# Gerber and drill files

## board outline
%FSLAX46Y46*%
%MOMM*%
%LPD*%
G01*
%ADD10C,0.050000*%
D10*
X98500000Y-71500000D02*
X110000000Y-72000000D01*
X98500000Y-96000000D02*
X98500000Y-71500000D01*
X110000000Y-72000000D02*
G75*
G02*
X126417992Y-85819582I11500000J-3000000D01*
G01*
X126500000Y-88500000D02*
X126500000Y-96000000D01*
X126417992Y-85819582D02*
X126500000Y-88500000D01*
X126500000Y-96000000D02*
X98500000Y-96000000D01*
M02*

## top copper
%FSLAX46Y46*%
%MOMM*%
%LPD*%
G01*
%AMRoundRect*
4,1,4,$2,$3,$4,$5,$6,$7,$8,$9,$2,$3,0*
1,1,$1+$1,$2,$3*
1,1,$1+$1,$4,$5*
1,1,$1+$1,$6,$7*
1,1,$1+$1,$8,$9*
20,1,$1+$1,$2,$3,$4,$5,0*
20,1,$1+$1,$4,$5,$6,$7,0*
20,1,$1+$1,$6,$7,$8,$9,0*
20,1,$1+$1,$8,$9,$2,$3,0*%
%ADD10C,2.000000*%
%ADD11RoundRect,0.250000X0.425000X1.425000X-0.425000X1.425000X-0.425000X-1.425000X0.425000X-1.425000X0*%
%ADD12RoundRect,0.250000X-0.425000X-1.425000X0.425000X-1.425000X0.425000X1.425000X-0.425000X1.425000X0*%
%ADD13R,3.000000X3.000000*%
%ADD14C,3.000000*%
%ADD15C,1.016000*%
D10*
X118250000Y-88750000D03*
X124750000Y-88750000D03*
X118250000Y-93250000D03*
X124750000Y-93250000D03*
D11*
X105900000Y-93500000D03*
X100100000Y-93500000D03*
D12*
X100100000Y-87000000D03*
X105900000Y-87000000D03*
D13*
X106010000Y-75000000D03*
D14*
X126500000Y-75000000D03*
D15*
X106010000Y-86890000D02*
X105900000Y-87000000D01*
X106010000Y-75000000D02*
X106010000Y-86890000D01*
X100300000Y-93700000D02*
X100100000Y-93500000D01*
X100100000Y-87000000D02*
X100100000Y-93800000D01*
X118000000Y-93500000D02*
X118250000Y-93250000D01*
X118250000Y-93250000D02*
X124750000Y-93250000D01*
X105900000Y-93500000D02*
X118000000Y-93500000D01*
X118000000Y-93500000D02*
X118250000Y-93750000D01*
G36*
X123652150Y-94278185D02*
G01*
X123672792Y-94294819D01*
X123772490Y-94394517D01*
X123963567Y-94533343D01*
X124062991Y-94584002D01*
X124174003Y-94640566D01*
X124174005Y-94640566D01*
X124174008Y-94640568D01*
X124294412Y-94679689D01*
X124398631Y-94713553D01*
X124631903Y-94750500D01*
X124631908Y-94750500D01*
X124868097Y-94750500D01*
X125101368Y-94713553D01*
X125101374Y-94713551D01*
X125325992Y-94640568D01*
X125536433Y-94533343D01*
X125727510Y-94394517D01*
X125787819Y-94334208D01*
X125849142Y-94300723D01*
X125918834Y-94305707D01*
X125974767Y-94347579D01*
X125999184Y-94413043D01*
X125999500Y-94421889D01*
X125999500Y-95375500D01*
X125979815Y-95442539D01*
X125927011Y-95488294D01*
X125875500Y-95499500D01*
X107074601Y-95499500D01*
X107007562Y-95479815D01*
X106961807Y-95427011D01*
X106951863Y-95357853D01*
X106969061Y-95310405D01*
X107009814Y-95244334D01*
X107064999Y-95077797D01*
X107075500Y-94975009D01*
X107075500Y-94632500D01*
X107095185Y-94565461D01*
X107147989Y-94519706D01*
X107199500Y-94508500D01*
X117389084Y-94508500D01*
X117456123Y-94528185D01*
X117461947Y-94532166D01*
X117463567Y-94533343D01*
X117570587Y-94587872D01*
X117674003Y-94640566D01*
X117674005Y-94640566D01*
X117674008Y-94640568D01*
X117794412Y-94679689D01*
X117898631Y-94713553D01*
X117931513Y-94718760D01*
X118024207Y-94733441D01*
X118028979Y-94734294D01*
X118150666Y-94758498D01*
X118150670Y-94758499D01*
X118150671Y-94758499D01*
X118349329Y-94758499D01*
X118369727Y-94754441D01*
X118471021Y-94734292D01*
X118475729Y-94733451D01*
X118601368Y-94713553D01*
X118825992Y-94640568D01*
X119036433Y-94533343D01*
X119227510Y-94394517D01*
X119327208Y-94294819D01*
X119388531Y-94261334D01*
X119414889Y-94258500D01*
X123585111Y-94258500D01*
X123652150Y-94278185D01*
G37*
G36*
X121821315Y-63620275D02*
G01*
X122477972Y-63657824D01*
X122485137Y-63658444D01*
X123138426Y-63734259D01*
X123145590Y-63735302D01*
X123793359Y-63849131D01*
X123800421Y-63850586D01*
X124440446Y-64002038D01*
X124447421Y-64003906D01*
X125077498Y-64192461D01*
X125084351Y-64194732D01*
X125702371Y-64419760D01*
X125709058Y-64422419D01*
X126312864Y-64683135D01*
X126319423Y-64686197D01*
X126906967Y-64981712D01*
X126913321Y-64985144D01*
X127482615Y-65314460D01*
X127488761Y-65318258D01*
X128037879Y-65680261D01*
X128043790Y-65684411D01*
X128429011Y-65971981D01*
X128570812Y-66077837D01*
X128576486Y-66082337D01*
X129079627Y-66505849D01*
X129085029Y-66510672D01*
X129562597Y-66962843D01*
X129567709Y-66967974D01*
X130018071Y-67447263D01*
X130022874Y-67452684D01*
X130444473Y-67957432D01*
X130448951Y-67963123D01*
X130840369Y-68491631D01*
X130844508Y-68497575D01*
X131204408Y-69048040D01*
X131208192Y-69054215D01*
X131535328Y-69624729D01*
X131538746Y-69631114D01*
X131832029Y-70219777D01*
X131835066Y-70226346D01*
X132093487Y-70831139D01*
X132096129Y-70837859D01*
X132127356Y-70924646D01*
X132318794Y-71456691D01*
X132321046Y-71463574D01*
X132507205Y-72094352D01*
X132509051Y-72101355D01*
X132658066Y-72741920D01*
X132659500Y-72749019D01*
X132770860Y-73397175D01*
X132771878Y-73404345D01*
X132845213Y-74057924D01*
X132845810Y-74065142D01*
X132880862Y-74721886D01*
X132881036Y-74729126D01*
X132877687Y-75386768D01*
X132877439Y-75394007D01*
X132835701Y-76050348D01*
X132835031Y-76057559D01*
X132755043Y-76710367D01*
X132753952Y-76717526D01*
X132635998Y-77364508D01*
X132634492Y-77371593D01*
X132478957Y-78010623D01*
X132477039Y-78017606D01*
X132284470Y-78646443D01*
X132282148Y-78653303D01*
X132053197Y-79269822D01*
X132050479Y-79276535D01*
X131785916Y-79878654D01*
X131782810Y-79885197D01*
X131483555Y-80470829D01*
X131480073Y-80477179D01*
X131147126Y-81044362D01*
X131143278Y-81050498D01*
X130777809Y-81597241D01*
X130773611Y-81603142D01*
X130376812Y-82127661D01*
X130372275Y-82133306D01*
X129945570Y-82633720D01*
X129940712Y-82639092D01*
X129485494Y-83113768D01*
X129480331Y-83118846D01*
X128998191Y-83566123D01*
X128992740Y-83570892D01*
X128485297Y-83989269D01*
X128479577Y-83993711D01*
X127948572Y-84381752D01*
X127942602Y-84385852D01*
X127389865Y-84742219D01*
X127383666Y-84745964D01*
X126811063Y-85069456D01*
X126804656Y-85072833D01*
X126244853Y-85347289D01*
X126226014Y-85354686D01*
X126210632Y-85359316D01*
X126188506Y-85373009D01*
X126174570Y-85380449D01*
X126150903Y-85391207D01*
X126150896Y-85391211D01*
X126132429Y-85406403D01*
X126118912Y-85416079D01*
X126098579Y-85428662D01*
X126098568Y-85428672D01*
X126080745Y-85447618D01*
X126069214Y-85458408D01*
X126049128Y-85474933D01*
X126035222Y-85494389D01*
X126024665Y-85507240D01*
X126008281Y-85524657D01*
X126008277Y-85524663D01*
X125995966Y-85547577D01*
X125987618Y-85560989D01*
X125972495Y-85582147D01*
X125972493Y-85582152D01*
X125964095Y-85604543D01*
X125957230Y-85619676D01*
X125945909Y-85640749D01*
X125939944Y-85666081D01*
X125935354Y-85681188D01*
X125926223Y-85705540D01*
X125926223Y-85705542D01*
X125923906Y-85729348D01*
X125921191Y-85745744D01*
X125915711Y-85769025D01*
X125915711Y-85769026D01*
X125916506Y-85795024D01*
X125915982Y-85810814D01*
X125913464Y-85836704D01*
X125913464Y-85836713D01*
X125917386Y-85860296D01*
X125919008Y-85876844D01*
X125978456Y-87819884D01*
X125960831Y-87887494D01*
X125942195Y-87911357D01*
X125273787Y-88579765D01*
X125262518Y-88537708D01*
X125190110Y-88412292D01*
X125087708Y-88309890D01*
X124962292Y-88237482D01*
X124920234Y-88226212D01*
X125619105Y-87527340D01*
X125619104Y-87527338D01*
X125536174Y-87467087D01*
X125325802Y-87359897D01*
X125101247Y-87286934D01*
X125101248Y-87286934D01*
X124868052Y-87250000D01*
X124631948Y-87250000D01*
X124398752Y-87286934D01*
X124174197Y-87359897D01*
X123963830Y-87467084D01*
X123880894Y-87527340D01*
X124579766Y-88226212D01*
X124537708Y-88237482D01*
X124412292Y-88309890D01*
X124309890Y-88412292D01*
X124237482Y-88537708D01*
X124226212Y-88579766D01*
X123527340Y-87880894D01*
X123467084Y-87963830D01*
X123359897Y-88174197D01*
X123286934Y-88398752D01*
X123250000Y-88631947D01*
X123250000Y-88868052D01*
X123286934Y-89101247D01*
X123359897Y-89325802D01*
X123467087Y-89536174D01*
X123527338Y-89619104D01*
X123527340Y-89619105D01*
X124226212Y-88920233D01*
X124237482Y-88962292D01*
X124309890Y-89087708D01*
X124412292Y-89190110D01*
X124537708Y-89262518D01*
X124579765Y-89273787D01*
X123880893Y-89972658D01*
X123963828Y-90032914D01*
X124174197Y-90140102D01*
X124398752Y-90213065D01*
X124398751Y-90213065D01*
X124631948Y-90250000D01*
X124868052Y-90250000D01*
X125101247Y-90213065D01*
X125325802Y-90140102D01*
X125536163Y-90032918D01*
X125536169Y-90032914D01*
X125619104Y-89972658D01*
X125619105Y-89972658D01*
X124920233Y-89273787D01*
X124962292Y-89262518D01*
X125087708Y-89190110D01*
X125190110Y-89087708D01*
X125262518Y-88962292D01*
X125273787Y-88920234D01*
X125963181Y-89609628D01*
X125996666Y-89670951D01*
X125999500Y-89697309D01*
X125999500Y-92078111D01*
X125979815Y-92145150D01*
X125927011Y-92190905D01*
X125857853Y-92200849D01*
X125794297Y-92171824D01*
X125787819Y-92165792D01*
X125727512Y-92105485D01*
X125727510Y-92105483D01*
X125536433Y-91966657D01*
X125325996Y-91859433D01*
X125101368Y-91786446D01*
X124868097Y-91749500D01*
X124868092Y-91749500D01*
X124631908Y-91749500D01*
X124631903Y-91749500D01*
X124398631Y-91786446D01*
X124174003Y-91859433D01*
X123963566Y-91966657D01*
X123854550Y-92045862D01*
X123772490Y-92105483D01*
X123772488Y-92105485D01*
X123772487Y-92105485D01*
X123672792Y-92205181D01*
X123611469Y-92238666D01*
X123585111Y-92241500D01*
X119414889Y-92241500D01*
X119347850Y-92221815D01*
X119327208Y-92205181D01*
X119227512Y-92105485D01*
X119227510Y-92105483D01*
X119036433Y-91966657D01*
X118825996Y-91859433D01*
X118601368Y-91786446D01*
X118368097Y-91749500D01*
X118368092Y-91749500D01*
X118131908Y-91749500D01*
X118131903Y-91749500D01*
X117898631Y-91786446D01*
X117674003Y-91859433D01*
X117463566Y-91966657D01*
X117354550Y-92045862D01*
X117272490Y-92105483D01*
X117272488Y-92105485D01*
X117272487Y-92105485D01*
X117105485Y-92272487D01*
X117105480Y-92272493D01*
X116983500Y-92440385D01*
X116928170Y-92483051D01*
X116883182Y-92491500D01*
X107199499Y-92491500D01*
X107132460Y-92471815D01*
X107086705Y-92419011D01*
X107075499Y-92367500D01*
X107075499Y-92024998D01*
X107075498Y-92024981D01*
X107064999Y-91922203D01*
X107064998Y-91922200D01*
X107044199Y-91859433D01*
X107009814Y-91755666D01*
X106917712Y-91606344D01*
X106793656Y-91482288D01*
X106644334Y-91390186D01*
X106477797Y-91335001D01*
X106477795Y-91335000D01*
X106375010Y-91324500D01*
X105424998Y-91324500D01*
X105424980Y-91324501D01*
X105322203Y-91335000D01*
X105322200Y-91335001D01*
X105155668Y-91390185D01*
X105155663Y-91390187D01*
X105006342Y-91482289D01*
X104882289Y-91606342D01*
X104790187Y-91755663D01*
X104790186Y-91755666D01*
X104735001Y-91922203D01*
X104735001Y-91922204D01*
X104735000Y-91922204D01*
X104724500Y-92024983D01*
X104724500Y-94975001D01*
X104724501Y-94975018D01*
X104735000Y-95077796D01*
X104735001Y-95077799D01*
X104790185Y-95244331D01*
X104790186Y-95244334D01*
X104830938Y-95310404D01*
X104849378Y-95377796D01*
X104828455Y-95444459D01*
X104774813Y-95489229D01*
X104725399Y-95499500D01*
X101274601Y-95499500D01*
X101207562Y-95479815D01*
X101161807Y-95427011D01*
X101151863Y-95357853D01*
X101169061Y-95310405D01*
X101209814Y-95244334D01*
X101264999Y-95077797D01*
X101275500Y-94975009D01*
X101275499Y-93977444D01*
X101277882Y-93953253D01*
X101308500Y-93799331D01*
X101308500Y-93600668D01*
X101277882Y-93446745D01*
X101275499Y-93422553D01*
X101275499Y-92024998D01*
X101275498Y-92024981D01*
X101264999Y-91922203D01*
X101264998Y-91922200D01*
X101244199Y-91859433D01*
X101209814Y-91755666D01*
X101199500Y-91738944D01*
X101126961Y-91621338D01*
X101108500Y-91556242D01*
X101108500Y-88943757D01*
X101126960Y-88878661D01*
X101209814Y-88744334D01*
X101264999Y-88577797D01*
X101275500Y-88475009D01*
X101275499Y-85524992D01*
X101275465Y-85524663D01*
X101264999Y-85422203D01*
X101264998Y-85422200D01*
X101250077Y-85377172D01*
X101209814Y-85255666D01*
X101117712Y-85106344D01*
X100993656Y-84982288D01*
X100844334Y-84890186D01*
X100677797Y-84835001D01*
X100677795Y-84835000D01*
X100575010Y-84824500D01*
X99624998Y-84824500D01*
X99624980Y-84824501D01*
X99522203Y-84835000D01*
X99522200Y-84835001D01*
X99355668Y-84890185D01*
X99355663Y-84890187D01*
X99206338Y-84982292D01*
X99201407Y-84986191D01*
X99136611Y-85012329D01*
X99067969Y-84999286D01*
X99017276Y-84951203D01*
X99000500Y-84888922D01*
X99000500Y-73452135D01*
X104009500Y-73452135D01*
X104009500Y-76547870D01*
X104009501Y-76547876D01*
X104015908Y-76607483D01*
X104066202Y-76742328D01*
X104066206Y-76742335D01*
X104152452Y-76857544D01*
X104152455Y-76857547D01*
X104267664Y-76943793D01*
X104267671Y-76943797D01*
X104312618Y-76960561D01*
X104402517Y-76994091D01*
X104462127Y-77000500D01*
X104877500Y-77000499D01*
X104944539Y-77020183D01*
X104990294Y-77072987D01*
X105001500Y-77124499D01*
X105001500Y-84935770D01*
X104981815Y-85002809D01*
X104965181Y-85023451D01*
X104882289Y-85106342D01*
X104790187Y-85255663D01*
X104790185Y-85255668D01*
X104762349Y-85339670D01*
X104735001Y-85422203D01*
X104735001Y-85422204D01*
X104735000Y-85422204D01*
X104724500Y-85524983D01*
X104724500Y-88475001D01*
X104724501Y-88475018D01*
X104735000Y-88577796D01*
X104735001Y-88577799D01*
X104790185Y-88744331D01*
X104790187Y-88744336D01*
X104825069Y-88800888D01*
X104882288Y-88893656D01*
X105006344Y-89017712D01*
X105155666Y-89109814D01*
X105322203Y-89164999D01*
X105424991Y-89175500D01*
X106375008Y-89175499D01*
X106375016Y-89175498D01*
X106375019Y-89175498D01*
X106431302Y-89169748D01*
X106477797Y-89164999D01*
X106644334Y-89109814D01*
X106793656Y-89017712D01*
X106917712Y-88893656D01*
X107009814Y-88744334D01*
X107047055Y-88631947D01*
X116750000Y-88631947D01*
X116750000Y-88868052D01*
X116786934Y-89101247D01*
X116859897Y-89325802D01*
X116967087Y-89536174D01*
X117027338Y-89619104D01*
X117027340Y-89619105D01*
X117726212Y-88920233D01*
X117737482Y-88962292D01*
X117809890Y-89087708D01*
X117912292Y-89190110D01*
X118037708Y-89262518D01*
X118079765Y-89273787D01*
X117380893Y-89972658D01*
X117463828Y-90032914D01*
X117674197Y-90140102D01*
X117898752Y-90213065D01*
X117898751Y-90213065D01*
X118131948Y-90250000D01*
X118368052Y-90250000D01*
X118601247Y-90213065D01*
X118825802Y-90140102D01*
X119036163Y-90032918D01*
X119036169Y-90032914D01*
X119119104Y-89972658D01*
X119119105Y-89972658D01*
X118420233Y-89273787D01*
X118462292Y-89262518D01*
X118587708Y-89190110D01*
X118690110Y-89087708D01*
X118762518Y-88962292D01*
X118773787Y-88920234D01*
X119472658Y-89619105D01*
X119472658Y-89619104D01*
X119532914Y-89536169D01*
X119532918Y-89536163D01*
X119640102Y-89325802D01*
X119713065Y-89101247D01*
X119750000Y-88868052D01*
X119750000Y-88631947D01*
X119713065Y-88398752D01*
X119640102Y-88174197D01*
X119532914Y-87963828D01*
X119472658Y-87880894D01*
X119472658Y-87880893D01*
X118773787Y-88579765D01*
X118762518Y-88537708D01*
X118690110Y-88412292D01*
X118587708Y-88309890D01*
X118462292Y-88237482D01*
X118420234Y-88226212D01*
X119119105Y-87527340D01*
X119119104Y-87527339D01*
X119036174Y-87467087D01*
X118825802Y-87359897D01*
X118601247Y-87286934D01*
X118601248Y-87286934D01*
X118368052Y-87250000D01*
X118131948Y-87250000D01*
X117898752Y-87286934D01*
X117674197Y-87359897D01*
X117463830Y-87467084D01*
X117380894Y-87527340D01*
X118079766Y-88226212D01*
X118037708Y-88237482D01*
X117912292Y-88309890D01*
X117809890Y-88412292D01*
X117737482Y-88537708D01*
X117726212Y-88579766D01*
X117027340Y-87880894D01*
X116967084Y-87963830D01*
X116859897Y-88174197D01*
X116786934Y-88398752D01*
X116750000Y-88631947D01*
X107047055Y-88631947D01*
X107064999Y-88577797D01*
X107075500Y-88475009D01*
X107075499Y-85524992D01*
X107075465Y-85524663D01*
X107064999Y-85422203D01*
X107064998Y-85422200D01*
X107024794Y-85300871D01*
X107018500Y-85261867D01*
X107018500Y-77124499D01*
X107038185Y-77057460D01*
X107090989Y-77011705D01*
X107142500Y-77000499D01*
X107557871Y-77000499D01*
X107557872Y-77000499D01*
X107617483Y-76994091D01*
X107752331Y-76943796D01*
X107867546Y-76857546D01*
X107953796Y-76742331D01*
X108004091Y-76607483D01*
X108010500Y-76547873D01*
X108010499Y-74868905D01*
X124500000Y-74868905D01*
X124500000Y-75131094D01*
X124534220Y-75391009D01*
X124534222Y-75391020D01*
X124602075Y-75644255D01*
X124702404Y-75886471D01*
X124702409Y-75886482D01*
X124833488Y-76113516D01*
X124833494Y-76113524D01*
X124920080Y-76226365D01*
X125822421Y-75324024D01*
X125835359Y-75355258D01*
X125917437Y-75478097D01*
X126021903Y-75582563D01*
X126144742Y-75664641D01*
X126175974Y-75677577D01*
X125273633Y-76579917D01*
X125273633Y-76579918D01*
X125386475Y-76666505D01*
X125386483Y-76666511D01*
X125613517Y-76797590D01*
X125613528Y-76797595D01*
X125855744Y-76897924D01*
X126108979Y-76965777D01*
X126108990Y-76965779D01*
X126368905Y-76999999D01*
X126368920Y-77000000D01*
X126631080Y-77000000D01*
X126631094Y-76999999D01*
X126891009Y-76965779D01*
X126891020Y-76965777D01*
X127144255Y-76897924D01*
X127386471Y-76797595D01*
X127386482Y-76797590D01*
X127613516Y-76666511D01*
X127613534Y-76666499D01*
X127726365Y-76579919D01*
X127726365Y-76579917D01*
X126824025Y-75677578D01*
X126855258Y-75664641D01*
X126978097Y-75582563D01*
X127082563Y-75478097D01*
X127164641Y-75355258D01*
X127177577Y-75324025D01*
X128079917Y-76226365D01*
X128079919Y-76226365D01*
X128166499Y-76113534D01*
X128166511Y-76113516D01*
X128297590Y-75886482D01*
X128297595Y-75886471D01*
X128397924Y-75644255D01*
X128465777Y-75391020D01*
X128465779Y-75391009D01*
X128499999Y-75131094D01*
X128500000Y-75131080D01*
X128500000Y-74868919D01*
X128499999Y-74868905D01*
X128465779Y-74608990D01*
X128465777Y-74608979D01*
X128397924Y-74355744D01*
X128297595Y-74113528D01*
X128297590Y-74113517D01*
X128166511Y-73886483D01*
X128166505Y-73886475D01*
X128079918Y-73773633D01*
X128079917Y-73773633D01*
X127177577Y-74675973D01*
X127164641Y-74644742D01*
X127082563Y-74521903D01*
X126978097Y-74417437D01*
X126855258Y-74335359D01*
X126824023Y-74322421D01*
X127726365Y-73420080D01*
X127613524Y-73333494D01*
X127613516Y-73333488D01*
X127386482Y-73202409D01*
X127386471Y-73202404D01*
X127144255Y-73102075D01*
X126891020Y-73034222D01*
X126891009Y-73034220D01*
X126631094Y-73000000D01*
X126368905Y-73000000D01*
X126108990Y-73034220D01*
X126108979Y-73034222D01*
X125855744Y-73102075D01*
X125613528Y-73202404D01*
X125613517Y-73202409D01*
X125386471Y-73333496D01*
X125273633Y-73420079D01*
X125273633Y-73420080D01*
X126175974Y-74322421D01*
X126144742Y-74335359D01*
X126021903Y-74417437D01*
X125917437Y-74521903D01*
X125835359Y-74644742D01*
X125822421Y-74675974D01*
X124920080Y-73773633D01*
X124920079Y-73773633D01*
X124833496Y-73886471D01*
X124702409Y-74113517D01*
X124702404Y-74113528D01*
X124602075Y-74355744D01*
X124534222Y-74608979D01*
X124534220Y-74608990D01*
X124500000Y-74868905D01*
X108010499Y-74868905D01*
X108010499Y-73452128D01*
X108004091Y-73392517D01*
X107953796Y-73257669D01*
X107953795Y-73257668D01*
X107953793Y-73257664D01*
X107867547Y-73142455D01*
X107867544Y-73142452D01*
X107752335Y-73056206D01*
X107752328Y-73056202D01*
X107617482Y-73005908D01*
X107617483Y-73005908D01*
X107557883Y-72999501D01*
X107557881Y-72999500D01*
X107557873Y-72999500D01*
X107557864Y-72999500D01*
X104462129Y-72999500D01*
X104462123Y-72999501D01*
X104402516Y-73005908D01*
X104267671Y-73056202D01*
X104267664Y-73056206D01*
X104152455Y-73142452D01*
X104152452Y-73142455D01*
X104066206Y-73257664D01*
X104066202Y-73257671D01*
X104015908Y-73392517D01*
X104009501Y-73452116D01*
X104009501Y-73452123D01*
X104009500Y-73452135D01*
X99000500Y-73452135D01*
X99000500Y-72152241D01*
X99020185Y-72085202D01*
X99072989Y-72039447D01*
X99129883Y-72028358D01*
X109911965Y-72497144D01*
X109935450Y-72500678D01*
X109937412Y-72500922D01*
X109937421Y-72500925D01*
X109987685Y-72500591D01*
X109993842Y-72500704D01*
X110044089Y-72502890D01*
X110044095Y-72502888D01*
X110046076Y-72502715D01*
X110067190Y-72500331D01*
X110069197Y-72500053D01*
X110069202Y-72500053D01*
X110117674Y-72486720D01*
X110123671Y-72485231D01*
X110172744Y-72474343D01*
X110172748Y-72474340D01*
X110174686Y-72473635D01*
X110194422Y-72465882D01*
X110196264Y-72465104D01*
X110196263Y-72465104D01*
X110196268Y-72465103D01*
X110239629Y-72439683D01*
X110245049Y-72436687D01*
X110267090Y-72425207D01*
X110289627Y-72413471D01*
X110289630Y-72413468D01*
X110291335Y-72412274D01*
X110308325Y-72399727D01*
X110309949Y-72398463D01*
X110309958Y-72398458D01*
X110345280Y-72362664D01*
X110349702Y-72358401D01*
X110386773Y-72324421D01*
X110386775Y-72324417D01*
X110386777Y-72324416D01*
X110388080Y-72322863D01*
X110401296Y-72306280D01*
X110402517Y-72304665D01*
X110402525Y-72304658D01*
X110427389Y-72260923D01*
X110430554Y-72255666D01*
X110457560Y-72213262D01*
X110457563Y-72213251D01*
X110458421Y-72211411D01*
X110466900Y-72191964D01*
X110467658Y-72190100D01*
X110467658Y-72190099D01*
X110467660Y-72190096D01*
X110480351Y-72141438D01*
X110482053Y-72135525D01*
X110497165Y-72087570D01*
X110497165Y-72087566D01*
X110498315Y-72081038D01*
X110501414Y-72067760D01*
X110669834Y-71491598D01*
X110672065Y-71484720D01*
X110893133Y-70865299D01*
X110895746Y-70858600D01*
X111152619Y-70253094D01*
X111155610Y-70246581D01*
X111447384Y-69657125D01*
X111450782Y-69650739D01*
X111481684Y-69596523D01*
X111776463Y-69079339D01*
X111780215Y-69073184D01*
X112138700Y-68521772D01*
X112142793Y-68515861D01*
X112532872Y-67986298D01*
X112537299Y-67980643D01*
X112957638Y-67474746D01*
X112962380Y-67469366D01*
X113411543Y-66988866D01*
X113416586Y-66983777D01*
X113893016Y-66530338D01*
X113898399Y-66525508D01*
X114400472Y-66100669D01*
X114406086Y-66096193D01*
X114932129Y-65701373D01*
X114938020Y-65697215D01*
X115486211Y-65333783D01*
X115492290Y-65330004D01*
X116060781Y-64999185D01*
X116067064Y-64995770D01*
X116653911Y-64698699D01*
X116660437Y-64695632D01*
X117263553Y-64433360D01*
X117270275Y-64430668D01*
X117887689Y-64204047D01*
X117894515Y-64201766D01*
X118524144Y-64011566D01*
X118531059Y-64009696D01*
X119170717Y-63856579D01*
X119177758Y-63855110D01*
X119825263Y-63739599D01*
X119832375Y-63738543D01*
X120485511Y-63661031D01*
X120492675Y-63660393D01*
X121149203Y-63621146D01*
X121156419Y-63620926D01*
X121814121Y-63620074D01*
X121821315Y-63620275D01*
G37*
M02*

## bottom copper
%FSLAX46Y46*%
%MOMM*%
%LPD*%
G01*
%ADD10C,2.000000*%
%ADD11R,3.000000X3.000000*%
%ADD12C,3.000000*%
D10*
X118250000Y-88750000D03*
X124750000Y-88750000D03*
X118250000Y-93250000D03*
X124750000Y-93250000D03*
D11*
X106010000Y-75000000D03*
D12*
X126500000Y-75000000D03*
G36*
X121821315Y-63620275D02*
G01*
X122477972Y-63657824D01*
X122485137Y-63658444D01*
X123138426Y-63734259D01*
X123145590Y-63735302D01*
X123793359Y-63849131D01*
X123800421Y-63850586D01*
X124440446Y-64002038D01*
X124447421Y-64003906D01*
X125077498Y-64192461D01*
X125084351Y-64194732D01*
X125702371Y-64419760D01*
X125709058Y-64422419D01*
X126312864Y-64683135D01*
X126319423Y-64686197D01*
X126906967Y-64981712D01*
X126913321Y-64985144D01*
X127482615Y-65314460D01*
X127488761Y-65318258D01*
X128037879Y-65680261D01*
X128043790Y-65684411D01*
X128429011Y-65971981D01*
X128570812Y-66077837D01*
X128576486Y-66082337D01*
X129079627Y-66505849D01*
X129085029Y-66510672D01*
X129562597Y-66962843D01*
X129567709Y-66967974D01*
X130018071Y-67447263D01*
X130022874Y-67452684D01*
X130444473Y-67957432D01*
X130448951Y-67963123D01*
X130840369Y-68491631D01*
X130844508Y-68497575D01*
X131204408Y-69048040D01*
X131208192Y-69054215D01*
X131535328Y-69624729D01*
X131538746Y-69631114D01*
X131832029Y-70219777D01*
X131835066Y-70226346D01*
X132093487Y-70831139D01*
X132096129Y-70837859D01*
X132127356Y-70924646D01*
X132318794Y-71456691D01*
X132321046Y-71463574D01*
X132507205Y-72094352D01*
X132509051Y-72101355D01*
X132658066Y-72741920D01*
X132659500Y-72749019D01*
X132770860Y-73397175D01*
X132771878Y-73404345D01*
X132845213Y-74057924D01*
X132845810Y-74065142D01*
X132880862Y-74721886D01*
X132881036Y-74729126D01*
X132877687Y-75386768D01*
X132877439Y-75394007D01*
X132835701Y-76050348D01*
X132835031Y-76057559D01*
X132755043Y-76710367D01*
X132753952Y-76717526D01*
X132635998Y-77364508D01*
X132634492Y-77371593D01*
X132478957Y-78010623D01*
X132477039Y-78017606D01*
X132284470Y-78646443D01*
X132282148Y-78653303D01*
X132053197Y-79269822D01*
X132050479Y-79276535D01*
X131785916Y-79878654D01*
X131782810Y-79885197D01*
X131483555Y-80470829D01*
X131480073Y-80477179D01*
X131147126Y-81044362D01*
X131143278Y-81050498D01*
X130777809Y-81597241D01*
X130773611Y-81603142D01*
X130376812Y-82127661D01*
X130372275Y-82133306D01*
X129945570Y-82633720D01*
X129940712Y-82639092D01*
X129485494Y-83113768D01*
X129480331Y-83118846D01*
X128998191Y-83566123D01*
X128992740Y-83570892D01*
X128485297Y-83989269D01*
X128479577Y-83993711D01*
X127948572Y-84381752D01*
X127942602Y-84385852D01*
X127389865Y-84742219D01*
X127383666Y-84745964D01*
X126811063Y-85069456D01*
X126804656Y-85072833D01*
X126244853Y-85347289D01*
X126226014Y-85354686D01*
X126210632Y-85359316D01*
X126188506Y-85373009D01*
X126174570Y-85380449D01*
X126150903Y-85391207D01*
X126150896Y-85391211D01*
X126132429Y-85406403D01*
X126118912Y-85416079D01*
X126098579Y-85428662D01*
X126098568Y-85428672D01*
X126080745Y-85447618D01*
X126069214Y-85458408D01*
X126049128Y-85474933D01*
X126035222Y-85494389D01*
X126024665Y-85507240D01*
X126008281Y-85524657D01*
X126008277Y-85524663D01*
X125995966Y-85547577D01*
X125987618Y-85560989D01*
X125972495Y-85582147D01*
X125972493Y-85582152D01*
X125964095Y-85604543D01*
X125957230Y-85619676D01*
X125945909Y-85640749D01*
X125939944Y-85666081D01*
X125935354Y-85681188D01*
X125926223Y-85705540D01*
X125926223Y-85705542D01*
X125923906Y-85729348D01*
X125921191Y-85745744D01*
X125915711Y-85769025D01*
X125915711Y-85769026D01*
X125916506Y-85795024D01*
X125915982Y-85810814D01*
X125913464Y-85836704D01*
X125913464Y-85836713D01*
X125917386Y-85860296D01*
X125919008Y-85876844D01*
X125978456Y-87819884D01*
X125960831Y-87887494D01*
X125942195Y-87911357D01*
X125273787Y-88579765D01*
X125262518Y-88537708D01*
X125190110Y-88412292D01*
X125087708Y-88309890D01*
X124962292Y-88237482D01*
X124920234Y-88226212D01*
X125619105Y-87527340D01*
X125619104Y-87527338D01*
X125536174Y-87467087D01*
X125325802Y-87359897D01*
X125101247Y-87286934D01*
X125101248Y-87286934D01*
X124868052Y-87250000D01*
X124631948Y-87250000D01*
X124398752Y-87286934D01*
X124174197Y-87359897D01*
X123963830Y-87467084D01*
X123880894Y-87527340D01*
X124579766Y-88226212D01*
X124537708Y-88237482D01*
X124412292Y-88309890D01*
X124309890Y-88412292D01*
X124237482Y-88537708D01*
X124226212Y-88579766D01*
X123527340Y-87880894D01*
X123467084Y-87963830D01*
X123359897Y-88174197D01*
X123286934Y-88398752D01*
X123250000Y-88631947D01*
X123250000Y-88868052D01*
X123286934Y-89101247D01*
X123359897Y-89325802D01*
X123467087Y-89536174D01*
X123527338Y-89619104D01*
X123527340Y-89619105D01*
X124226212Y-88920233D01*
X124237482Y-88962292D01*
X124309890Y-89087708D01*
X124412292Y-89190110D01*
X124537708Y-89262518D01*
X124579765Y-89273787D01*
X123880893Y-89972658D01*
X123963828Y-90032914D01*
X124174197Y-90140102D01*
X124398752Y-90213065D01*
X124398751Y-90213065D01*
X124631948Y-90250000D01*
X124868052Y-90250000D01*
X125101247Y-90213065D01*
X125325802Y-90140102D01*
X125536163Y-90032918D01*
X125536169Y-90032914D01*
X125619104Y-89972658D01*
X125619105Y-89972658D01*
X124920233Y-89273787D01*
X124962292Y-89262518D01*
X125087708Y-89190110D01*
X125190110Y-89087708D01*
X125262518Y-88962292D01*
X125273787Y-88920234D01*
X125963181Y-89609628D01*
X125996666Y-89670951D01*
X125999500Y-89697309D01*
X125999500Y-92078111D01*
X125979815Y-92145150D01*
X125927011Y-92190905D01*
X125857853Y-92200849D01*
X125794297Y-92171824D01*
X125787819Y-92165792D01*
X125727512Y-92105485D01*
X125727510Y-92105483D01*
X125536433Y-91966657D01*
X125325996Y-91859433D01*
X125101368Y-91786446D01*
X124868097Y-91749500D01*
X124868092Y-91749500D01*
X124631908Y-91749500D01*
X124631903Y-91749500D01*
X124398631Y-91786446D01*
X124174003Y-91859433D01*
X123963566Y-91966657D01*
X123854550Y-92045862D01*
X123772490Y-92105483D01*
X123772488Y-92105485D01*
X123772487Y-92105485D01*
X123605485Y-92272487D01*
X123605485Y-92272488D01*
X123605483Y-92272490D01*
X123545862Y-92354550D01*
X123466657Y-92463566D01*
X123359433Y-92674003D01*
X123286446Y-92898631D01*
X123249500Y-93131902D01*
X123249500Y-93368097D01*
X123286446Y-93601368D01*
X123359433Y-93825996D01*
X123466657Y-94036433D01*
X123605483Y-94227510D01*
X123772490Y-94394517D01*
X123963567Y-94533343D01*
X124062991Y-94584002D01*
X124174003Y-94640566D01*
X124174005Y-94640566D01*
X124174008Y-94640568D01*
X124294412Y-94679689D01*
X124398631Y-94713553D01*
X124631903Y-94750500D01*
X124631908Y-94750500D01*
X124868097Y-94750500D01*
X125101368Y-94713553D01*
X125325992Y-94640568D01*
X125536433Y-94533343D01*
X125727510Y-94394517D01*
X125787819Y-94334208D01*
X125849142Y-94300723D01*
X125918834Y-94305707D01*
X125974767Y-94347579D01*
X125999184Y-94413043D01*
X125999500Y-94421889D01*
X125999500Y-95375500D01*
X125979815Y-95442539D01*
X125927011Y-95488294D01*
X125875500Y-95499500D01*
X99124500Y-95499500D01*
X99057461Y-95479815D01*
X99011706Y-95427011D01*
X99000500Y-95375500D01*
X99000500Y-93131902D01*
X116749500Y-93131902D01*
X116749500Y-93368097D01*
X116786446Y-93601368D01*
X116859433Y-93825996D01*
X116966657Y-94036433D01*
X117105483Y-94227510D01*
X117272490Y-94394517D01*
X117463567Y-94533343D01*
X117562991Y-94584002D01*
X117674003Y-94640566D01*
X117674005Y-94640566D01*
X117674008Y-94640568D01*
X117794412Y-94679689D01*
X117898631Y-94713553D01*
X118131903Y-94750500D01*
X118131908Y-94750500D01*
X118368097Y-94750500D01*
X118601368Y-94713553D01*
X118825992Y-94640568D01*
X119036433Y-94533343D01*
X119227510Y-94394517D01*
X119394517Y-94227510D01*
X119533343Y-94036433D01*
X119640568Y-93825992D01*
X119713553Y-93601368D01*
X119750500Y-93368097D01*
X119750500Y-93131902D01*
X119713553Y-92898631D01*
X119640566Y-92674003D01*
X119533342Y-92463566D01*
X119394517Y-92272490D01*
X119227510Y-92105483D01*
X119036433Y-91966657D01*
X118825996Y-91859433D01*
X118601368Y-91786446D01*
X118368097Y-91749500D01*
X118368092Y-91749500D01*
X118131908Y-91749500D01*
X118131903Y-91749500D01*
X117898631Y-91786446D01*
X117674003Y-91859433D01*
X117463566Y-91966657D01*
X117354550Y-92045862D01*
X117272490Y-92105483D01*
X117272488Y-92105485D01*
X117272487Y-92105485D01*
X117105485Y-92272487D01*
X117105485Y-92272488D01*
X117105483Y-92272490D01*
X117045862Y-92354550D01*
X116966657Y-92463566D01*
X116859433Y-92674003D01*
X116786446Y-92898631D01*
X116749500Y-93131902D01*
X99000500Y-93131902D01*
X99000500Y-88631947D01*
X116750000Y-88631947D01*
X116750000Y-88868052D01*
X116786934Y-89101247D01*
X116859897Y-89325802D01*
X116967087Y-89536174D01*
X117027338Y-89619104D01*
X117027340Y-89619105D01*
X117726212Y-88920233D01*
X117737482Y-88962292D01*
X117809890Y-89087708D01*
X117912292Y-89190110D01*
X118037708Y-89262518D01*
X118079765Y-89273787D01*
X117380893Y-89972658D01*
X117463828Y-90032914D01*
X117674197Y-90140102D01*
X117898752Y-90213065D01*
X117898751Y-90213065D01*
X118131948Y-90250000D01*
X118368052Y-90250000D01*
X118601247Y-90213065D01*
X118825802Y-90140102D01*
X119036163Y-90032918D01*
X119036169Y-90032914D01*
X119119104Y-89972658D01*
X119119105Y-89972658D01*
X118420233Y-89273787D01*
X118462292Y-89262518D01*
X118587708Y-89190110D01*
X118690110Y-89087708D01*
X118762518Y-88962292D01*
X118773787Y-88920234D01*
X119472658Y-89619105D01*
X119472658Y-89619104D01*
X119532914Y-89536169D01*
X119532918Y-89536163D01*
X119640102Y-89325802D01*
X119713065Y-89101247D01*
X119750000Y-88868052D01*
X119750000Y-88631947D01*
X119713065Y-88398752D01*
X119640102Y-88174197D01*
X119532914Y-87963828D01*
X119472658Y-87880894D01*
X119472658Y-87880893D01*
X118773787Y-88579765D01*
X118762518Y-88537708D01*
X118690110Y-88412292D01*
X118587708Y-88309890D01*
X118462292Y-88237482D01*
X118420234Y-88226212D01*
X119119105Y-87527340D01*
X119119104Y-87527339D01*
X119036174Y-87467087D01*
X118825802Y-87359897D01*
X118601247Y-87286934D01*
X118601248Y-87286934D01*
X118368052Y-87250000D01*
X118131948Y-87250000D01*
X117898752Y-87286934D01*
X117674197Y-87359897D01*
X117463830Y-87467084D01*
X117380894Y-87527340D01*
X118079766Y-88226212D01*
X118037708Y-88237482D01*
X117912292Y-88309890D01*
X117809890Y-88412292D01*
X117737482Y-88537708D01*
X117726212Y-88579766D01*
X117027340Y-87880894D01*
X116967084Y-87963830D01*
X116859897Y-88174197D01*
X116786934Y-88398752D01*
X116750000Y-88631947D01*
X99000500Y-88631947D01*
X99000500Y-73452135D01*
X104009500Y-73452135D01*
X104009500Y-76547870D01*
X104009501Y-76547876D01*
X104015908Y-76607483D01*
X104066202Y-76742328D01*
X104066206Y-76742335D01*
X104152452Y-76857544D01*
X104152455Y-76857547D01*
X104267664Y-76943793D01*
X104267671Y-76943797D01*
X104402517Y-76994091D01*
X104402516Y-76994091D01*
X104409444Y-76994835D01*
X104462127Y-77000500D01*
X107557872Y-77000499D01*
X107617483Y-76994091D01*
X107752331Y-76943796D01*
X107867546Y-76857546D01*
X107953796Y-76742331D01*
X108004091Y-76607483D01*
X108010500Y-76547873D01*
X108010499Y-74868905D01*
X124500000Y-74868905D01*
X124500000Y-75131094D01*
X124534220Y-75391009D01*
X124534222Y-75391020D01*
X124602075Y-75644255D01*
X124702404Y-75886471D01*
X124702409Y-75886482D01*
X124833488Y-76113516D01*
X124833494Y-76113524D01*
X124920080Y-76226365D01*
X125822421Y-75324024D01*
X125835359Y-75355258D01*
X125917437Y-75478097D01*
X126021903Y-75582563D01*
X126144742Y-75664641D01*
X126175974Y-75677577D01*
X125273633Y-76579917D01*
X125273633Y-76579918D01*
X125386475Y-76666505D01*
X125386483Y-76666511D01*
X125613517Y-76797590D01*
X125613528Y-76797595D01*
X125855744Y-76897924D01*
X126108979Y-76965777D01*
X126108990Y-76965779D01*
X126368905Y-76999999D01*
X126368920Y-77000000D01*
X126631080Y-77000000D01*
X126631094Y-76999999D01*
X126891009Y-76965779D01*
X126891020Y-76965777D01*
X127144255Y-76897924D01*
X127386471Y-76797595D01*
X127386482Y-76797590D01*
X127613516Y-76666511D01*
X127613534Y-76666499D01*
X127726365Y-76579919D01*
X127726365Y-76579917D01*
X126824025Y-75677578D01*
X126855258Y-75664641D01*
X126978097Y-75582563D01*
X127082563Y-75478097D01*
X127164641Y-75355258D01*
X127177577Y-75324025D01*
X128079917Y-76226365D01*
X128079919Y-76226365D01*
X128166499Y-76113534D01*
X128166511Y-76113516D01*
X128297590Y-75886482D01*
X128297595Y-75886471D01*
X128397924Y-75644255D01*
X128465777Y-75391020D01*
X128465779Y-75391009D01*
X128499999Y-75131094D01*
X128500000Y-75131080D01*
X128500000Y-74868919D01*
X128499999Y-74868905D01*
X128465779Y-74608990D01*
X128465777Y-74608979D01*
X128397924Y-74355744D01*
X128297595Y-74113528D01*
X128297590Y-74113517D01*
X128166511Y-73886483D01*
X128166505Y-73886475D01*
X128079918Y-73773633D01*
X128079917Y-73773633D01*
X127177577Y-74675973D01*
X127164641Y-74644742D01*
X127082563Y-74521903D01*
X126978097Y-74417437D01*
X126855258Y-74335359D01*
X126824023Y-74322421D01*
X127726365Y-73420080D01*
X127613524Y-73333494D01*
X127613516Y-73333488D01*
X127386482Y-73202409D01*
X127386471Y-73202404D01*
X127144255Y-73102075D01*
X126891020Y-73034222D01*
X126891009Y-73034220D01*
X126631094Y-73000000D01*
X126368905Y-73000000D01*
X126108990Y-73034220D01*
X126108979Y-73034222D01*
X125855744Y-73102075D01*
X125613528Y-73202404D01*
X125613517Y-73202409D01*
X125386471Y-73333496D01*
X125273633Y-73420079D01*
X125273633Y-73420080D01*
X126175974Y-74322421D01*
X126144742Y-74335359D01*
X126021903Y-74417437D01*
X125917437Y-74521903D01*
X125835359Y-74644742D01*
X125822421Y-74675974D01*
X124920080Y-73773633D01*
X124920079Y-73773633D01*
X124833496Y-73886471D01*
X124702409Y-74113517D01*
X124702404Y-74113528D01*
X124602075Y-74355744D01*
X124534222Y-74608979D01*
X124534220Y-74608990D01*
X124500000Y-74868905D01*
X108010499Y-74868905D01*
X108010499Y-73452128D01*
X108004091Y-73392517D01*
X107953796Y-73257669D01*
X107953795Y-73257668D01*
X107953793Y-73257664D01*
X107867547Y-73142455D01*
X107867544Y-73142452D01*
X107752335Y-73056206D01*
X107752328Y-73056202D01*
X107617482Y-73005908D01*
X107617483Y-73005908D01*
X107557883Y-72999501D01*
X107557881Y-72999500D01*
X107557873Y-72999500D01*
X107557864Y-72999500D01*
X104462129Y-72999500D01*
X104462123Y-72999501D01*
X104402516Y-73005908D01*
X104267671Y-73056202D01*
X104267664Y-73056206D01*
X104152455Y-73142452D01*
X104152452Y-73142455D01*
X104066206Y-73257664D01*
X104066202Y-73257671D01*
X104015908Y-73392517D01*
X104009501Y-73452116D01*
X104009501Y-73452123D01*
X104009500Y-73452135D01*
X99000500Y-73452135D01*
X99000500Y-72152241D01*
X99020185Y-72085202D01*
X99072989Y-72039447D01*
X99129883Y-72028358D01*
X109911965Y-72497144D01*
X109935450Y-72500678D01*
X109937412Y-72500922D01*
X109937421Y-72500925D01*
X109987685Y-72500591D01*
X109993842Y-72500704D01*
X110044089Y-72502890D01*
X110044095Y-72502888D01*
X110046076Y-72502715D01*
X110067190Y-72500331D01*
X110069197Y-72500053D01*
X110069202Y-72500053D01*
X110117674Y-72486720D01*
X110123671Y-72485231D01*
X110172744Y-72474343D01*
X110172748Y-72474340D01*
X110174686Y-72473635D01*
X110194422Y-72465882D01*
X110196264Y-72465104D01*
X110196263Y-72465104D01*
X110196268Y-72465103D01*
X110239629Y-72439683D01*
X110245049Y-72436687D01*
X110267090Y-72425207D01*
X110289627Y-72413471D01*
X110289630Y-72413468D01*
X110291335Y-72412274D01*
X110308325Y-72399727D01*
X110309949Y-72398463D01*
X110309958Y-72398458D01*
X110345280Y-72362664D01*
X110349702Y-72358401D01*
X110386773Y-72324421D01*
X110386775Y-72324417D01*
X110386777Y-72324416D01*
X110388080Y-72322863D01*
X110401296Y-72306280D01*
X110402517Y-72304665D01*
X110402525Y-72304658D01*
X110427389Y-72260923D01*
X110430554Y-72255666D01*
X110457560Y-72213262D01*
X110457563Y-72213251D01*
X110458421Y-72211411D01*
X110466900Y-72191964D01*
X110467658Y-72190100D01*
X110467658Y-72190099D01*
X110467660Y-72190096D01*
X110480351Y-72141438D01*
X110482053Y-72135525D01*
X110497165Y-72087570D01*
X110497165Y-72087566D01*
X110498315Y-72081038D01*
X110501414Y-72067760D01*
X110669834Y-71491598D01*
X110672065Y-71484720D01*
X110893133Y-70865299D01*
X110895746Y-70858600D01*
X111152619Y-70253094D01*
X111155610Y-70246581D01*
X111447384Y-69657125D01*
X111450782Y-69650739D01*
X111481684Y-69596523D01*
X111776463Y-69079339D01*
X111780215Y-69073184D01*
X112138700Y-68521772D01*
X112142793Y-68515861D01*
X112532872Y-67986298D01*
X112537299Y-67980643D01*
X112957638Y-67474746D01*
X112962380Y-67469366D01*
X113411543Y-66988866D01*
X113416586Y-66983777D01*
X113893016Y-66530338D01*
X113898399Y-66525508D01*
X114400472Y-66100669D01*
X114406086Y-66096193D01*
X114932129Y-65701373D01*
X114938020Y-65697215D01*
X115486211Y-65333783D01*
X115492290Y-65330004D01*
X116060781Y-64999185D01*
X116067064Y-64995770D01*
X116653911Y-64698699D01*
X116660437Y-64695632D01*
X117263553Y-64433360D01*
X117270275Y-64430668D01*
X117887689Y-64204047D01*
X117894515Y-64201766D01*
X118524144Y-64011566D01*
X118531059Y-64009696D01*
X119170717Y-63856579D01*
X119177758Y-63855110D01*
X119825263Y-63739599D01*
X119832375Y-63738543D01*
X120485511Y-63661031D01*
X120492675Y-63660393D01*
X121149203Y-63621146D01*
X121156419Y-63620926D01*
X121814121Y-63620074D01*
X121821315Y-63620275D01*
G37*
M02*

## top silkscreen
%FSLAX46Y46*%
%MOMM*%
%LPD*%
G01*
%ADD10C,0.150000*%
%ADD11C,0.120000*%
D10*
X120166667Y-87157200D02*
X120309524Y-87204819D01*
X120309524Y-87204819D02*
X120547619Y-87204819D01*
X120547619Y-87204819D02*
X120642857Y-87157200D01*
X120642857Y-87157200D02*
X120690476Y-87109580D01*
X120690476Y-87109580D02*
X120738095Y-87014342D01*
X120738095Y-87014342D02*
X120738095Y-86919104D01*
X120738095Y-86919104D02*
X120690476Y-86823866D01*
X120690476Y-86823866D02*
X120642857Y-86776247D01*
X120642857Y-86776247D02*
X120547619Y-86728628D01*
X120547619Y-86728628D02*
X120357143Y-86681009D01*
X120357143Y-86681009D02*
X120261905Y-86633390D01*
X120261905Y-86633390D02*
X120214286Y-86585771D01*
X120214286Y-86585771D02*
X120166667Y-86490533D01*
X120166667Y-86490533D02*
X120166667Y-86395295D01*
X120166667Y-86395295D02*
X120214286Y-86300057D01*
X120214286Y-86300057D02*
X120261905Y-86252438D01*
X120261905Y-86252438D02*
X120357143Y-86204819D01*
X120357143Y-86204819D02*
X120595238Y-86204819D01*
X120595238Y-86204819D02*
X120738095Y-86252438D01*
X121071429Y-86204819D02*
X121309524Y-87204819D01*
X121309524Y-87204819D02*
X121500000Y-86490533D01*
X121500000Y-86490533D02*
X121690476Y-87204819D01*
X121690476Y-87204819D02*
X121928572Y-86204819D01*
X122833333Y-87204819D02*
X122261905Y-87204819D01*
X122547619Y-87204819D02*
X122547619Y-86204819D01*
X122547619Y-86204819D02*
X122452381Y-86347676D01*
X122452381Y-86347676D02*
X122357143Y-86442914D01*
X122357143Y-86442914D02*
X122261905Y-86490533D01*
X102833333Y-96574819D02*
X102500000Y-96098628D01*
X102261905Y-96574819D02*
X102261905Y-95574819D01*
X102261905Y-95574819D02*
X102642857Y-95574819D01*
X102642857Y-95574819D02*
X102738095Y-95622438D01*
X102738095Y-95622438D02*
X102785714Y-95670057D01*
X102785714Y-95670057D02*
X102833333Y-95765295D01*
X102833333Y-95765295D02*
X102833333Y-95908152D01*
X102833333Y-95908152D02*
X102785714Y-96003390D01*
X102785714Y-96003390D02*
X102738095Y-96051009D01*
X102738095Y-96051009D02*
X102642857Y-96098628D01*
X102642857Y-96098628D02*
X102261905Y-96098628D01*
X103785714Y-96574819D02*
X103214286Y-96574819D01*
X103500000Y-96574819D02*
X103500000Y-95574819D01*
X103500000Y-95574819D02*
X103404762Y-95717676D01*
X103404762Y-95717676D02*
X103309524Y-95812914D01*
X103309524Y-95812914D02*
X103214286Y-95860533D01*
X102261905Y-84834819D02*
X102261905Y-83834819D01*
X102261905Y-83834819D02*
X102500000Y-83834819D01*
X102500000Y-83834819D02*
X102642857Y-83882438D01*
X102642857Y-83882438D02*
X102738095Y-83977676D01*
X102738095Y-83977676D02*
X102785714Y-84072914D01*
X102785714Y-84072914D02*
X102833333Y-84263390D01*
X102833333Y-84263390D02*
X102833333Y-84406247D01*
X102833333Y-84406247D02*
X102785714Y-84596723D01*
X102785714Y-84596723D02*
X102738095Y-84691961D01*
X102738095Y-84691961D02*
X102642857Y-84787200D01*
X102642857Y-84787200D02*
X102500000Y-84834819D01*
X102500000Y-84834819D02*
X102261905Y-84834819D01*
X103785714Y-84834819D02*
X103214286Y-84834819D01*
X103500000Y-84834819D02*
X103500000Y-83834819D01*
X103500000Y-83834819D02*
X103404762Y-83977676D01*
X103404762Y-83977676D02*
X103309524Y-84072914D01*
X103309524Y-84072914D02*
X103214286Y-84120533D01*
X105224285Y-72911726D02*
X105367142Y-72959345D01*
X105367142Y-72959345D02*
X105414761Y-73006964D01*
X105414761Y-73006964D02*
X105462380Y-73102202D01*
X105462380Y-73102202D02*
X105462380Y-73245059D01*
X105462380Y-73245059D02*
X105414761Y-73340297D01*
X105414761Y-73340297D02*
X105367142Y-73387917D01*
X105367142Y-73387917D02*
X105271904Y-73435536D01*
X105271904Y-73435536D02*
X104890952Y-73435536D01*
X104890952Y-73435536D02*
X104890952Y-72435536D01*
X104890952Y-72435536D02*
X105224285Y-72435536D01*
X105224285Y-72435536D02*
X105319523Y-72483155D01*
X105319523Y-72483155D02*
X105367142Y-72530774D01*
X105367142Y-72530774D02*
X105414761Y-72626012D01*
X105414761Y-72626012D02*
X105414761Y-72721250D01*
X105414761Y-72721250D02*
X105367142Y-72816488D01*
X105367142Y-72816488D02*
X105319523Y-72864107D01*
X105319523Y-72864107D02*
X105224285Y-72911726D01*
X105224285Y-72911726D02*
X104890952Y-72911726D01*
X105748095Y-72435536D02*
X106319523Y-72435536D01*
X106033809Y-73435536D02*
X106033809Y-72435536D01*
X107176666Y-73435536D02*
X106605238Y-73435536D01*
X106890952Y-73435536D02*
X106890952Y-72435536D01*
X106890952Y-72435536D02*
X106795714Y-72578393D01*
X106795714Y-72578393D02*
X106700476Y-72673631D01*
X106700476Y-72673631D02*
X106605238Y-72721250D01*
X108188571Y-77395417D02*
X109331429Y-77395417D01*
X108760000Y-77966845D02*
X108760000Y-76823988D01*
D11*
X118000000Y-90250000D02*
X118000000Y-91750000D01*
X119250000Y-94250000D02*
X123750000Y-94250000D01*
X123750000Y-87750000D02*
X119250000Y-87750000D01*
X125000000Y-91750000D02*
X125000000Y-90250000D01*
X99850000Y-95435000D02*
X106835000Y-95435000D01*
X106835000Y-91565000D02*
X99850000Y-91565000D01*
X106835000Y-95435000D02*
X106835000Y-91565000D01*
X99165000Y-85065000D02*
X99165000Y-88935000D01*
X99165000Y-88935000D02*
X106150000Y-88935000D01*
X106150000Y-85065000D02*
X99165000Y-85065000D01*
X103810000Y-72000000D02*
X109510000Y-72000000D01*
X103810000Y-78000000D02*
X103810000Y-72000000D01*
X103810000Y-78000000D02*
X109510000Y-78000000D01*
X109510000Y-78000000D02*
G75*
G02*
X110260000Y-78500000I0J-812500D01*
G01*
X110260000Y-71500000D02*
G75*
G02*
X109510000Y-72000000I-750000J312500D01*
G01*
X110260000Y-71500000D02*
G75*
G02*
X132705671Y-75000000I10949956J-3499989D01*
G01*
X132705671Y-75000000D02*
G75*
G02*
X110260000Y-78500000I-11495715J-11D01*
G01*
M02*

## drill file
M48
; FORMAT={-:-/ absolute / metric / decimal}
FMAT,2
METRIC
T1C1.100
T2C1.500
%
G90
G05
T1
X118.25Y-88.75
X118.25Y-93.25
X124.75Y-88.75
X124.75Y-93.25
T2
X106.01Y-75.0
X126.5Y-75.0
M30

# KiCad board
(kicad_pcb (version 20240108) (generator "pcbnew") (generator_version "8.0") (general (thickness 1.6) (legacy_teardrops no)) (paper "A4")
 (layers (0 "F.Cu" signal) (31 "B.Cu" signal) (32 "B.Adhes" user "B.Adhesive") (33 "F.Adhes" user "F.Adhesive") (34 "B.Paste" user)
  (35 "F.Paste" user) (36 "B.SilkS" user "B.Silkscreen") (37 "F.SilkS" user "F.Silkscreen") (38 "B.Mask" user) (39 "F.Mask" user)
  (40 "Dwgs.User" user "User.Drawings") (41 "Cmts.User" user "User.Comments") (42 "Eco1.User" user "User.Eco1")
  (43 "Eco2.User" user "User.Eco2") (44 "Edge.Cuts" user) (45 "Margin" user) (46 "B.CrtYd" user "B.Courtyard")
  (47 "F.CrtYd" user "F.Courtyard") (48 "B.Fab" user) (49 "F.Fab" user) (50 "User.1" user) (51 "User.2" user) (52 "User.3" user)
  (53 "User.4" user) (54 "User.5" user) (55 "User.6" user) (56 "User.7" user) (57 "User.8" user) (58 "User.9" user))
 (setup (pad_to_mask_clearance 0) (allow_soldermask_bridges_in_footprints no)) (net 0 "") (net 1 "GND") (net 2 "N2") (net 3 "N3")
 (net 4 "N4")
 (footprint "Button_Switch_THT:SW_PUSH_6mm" (layer "F.Cu") (at 118.25 88.75)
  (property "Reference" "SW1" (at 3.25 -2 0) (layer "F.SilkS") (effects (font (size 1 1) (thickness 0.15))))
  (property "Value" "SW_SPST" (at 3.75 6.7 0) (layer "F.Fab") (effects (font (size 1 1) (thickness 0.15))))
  (fp_line (start -0.25 1.5) (end -0.25 3) (stroke (width 0.12) (type solid)) (layer "F.SilkS"))
  (fp_line (start 1 5.5) (end 5.5 5.5) (stroke (width 0.12) (type solid)) (layer "F.SilkS"))
  (fp_line (start 5.5 -1) (end 1 -1) (stroke (width 0.12) (type solid)) (layer "F.SilkS"))
  (fp_line (start 6.75 3) (end 6.75 1.5) (stroke (width 0.12) (type solid)) (layer "F.SilkS"))
  (pad "1" thru_hole circle (at 0 0 90) (size 2 2) (drill 1.1) (layers "*.Cu" "*.Mask") (remove_unused_layers no) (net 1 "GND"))
  (pad "1" thru_hole circle (at 6.5 0 90) (size 2 2) (drill 1.1) (layers "*.Cu" "*.Mask") (remove_unused_layers no) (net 1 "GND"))
  (pad "2" thru_hole circle (at 0 4.5 90) (size 2 2) (drill 1.1) (layers "*.Cu" "*.Mask") (remove_unused_layers no) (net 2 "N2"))
  (pad "2" thru_hole circle (at 6.5 4.5 90) (size 2 2) (drill 1.1) (layers "*.Cu" "*.Mask") (remove_unused_layers no) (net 2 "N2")))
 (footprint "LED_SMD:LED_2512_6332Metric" (layer "F.Cu") (at 103 93.5 180)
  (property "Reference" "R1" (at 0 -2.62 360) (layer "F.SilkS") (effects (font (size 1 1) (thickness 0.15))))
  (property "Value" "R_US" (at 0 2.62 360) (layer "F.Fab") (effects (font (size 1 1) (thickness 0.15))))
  (fp_line (start 3.15 -1.935) (end -3.835 -1.935) (stroke (width 0.12) (type solid)) (layer "F.SilkS"))
  (fp_line (start -3.835 1.935) (end 3.15 1.935) (stroke (width 0.12) (type solid)) (layer "F.SilkS"))
  (fp_line (start -3.835 -1.935) (end -3.835 1.935) (stroke (width 0.12) (type solid)) (layer "F.SilkS"))
  (pad "1" smd roundrect (at -2.9 0 180) (size 1.35 3.35) (layers "F.Cu" "F.Paste" "F.Mask") (roundrect_rratio 0.185185) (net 2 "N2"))
  (pad "2" smd roundrect (at 2.9 0 180) (size 1.35 3.35) (layers "F.Cu" "F.Paste" "F.Mask") (roundrect_rratio 0.185185) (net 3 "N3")))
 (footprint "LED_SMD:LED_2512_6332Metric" (layer "F.Cu") (at 103 87)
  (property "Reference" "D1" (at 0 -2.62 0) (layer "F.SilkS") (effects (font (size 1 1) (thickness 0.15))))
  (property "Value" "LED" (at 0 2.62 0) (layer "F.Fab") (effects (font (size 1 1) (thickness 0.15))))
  (fp_line (start -3.835 -1.935) (end -3.835 1.935) (stroke (width 0.12) (type solid)) (layer "F.SilkS"))
  (fp_line (start -3.835 1.935) (end 3.15 1.935) (stroke (width 0.12) (type solid)) (layer "F.SilkS"))
  (fp_line (start 3.15 -1.935) (end -3.835 -1.935) (stroke (width 0.12) (type solid)) (layer "F.SilkS"))
  (pad "1" smd roundrect (at -2.9 0) (size 1.35 3.35) (layers "F.Cu" "F.Paste" "F.Mask") (roundrect_rratio 0.185185) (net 3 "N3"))
  (pad "2" smd roundrect (at 2.9 0) (size 1.35 3.35) (layers "F.Cu" "F.Paste" "F.Mask") (roundrect_rratio 0.185185) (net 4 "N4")))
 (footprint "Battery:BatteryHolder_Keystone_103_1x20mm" (layer "F.Cu") (at 106.01 75)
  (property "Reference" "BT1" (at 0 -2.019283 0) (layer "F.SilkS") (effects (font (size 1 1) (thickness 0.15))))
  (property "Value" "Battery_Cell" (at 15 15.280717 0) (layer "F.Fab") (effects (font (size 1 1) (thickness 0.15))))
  (fp_line (start -2.2 -3) (end 3.5 -3) (stroke (width 0.12) (type solid)) (layer "F.SilkS"))
  (fp_line (start -2.2 3) (end -2.2 -3) (stroke (width 0.12) (type solid)) (layer "F.SilkS"))
  (fp_line (start -2.2 3) (end 3.5 3) (stroke (width 0.12) (type solid)) (layer "F.SilkS"))
  (fp_arc (start 3.5 3) (mid 3.950694 3.136459) (end 4.25 3.5) (stroke (width 0.12) (type solid)) (layer "F.SilkS"))
  (fp_arc (start 4.25 -3.5) (mid 3.950694 -3.136459) (end 3.5 -3) (stroke (width 0.12) (type solid)) (layer "F.SilkS"))
  (fp_arc (start 4.25 -3.5) (mid 16.971103 -11.358466) (end 26.695671 0) (stroke (width 0.12) (type solid)) (layer "F.SilkS"))
  (fp_arc (start 26.695671 0) (mid 16.971103 11.358466) (end 4.25 3.5) (stroke (width 0.12) (type solid)) (layer "F.SilkS"))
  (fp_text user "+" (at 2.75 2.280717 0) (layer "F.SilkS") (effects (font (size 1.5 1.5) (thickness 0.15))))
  (pad "1" thru_hole rect (at 0 0) (size 3 3) (drill 1.5) (layers "*.Cu" "*.Mask") (remove_unused_layers no) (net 4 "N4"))
  (pad "2" thru_hole circle (at 20.49 0) (size 3 3) (drill 1.5) (layers "*.Cu" "*.Mask") (remove_unused_layers no) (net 1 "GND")))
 (gr_line (start 98.5 71.5) (end 110 72) (stroke (width 0.05) (type default)) (layer "Edge.Cuts"))
 (gr_line (start 98.5 96) (end 98.5 71.5) (stroke (width 0.05) (type default)) (layer "Edge.Cuts"))
 (gr_arc (start 110 72) (mid 129.153491 65.907471) (end 126.417992 85.819582) (stroke (width 0.05) (type default)) (layer "Edge.Cuts"))
 (gr_line (start 126.5 88.5) (end 126.5 96) (stroke (width 0.05) (type default)) (layer "Edge.Cuts"))
 (gr_line (start 126.417992 85.819582) (end 126.5 88.5) (stroke (width 0.05) (type default)) (layer "Edge.Cuts"))
 (gr_line (start 126.5 96) (end 98.5 96) (stroke (width 0.05) (type default)) (layer "Edge.Cuts"))
 (segment (start 106.01 86.89) (end 105.9 87) (width 1.016) (layer "F.Cu") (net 4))
 (segment (start 106.01 75) (end 106.01 86.89) (width 1.016) (layer "F.Cu") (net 4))
 (segment (start 100.3 93.7) (end 100.1 93.5) (width 1.016) (layer "F.Cu") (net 3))
 (segment (start 100.1 87) (end 100.1 93.8) (width 1.016) (layer "F.Cu") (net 3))
 (segment (start 118 93.5) (end 118.25 93.25) (width 1.016) (layer "F.Cu") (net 2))
 (segment (start 118.25 93.25) (end 124.75 93.25) (width 1.016) (layer "F.Cu") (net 2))
 (segment (start 105.9 93.5) (end 118 93.5) (width 1.016) (layer "F.Cu") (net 2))
 (segment (start 118 93.5) (end 118.25 93.75) (width 1.016) (layer "F.Cu") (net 2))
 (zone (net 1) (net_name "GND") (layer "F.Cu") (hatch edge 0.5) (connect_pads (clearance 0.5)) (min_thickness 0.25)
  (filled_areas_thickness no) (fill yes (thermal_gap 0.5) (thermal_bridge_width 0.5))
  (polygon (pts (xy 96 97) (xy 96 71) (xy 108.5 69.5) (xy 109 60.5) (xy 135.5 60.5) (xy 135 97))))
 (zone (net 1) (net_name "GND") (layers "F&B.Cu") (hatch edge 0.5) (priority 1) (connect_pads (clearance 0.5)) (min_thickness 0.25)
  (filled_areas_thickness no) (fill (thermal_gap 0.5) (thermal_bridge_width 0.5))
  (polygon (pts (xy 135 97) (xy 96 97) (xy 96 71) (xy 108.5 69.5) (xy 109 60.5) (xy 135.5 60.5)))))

